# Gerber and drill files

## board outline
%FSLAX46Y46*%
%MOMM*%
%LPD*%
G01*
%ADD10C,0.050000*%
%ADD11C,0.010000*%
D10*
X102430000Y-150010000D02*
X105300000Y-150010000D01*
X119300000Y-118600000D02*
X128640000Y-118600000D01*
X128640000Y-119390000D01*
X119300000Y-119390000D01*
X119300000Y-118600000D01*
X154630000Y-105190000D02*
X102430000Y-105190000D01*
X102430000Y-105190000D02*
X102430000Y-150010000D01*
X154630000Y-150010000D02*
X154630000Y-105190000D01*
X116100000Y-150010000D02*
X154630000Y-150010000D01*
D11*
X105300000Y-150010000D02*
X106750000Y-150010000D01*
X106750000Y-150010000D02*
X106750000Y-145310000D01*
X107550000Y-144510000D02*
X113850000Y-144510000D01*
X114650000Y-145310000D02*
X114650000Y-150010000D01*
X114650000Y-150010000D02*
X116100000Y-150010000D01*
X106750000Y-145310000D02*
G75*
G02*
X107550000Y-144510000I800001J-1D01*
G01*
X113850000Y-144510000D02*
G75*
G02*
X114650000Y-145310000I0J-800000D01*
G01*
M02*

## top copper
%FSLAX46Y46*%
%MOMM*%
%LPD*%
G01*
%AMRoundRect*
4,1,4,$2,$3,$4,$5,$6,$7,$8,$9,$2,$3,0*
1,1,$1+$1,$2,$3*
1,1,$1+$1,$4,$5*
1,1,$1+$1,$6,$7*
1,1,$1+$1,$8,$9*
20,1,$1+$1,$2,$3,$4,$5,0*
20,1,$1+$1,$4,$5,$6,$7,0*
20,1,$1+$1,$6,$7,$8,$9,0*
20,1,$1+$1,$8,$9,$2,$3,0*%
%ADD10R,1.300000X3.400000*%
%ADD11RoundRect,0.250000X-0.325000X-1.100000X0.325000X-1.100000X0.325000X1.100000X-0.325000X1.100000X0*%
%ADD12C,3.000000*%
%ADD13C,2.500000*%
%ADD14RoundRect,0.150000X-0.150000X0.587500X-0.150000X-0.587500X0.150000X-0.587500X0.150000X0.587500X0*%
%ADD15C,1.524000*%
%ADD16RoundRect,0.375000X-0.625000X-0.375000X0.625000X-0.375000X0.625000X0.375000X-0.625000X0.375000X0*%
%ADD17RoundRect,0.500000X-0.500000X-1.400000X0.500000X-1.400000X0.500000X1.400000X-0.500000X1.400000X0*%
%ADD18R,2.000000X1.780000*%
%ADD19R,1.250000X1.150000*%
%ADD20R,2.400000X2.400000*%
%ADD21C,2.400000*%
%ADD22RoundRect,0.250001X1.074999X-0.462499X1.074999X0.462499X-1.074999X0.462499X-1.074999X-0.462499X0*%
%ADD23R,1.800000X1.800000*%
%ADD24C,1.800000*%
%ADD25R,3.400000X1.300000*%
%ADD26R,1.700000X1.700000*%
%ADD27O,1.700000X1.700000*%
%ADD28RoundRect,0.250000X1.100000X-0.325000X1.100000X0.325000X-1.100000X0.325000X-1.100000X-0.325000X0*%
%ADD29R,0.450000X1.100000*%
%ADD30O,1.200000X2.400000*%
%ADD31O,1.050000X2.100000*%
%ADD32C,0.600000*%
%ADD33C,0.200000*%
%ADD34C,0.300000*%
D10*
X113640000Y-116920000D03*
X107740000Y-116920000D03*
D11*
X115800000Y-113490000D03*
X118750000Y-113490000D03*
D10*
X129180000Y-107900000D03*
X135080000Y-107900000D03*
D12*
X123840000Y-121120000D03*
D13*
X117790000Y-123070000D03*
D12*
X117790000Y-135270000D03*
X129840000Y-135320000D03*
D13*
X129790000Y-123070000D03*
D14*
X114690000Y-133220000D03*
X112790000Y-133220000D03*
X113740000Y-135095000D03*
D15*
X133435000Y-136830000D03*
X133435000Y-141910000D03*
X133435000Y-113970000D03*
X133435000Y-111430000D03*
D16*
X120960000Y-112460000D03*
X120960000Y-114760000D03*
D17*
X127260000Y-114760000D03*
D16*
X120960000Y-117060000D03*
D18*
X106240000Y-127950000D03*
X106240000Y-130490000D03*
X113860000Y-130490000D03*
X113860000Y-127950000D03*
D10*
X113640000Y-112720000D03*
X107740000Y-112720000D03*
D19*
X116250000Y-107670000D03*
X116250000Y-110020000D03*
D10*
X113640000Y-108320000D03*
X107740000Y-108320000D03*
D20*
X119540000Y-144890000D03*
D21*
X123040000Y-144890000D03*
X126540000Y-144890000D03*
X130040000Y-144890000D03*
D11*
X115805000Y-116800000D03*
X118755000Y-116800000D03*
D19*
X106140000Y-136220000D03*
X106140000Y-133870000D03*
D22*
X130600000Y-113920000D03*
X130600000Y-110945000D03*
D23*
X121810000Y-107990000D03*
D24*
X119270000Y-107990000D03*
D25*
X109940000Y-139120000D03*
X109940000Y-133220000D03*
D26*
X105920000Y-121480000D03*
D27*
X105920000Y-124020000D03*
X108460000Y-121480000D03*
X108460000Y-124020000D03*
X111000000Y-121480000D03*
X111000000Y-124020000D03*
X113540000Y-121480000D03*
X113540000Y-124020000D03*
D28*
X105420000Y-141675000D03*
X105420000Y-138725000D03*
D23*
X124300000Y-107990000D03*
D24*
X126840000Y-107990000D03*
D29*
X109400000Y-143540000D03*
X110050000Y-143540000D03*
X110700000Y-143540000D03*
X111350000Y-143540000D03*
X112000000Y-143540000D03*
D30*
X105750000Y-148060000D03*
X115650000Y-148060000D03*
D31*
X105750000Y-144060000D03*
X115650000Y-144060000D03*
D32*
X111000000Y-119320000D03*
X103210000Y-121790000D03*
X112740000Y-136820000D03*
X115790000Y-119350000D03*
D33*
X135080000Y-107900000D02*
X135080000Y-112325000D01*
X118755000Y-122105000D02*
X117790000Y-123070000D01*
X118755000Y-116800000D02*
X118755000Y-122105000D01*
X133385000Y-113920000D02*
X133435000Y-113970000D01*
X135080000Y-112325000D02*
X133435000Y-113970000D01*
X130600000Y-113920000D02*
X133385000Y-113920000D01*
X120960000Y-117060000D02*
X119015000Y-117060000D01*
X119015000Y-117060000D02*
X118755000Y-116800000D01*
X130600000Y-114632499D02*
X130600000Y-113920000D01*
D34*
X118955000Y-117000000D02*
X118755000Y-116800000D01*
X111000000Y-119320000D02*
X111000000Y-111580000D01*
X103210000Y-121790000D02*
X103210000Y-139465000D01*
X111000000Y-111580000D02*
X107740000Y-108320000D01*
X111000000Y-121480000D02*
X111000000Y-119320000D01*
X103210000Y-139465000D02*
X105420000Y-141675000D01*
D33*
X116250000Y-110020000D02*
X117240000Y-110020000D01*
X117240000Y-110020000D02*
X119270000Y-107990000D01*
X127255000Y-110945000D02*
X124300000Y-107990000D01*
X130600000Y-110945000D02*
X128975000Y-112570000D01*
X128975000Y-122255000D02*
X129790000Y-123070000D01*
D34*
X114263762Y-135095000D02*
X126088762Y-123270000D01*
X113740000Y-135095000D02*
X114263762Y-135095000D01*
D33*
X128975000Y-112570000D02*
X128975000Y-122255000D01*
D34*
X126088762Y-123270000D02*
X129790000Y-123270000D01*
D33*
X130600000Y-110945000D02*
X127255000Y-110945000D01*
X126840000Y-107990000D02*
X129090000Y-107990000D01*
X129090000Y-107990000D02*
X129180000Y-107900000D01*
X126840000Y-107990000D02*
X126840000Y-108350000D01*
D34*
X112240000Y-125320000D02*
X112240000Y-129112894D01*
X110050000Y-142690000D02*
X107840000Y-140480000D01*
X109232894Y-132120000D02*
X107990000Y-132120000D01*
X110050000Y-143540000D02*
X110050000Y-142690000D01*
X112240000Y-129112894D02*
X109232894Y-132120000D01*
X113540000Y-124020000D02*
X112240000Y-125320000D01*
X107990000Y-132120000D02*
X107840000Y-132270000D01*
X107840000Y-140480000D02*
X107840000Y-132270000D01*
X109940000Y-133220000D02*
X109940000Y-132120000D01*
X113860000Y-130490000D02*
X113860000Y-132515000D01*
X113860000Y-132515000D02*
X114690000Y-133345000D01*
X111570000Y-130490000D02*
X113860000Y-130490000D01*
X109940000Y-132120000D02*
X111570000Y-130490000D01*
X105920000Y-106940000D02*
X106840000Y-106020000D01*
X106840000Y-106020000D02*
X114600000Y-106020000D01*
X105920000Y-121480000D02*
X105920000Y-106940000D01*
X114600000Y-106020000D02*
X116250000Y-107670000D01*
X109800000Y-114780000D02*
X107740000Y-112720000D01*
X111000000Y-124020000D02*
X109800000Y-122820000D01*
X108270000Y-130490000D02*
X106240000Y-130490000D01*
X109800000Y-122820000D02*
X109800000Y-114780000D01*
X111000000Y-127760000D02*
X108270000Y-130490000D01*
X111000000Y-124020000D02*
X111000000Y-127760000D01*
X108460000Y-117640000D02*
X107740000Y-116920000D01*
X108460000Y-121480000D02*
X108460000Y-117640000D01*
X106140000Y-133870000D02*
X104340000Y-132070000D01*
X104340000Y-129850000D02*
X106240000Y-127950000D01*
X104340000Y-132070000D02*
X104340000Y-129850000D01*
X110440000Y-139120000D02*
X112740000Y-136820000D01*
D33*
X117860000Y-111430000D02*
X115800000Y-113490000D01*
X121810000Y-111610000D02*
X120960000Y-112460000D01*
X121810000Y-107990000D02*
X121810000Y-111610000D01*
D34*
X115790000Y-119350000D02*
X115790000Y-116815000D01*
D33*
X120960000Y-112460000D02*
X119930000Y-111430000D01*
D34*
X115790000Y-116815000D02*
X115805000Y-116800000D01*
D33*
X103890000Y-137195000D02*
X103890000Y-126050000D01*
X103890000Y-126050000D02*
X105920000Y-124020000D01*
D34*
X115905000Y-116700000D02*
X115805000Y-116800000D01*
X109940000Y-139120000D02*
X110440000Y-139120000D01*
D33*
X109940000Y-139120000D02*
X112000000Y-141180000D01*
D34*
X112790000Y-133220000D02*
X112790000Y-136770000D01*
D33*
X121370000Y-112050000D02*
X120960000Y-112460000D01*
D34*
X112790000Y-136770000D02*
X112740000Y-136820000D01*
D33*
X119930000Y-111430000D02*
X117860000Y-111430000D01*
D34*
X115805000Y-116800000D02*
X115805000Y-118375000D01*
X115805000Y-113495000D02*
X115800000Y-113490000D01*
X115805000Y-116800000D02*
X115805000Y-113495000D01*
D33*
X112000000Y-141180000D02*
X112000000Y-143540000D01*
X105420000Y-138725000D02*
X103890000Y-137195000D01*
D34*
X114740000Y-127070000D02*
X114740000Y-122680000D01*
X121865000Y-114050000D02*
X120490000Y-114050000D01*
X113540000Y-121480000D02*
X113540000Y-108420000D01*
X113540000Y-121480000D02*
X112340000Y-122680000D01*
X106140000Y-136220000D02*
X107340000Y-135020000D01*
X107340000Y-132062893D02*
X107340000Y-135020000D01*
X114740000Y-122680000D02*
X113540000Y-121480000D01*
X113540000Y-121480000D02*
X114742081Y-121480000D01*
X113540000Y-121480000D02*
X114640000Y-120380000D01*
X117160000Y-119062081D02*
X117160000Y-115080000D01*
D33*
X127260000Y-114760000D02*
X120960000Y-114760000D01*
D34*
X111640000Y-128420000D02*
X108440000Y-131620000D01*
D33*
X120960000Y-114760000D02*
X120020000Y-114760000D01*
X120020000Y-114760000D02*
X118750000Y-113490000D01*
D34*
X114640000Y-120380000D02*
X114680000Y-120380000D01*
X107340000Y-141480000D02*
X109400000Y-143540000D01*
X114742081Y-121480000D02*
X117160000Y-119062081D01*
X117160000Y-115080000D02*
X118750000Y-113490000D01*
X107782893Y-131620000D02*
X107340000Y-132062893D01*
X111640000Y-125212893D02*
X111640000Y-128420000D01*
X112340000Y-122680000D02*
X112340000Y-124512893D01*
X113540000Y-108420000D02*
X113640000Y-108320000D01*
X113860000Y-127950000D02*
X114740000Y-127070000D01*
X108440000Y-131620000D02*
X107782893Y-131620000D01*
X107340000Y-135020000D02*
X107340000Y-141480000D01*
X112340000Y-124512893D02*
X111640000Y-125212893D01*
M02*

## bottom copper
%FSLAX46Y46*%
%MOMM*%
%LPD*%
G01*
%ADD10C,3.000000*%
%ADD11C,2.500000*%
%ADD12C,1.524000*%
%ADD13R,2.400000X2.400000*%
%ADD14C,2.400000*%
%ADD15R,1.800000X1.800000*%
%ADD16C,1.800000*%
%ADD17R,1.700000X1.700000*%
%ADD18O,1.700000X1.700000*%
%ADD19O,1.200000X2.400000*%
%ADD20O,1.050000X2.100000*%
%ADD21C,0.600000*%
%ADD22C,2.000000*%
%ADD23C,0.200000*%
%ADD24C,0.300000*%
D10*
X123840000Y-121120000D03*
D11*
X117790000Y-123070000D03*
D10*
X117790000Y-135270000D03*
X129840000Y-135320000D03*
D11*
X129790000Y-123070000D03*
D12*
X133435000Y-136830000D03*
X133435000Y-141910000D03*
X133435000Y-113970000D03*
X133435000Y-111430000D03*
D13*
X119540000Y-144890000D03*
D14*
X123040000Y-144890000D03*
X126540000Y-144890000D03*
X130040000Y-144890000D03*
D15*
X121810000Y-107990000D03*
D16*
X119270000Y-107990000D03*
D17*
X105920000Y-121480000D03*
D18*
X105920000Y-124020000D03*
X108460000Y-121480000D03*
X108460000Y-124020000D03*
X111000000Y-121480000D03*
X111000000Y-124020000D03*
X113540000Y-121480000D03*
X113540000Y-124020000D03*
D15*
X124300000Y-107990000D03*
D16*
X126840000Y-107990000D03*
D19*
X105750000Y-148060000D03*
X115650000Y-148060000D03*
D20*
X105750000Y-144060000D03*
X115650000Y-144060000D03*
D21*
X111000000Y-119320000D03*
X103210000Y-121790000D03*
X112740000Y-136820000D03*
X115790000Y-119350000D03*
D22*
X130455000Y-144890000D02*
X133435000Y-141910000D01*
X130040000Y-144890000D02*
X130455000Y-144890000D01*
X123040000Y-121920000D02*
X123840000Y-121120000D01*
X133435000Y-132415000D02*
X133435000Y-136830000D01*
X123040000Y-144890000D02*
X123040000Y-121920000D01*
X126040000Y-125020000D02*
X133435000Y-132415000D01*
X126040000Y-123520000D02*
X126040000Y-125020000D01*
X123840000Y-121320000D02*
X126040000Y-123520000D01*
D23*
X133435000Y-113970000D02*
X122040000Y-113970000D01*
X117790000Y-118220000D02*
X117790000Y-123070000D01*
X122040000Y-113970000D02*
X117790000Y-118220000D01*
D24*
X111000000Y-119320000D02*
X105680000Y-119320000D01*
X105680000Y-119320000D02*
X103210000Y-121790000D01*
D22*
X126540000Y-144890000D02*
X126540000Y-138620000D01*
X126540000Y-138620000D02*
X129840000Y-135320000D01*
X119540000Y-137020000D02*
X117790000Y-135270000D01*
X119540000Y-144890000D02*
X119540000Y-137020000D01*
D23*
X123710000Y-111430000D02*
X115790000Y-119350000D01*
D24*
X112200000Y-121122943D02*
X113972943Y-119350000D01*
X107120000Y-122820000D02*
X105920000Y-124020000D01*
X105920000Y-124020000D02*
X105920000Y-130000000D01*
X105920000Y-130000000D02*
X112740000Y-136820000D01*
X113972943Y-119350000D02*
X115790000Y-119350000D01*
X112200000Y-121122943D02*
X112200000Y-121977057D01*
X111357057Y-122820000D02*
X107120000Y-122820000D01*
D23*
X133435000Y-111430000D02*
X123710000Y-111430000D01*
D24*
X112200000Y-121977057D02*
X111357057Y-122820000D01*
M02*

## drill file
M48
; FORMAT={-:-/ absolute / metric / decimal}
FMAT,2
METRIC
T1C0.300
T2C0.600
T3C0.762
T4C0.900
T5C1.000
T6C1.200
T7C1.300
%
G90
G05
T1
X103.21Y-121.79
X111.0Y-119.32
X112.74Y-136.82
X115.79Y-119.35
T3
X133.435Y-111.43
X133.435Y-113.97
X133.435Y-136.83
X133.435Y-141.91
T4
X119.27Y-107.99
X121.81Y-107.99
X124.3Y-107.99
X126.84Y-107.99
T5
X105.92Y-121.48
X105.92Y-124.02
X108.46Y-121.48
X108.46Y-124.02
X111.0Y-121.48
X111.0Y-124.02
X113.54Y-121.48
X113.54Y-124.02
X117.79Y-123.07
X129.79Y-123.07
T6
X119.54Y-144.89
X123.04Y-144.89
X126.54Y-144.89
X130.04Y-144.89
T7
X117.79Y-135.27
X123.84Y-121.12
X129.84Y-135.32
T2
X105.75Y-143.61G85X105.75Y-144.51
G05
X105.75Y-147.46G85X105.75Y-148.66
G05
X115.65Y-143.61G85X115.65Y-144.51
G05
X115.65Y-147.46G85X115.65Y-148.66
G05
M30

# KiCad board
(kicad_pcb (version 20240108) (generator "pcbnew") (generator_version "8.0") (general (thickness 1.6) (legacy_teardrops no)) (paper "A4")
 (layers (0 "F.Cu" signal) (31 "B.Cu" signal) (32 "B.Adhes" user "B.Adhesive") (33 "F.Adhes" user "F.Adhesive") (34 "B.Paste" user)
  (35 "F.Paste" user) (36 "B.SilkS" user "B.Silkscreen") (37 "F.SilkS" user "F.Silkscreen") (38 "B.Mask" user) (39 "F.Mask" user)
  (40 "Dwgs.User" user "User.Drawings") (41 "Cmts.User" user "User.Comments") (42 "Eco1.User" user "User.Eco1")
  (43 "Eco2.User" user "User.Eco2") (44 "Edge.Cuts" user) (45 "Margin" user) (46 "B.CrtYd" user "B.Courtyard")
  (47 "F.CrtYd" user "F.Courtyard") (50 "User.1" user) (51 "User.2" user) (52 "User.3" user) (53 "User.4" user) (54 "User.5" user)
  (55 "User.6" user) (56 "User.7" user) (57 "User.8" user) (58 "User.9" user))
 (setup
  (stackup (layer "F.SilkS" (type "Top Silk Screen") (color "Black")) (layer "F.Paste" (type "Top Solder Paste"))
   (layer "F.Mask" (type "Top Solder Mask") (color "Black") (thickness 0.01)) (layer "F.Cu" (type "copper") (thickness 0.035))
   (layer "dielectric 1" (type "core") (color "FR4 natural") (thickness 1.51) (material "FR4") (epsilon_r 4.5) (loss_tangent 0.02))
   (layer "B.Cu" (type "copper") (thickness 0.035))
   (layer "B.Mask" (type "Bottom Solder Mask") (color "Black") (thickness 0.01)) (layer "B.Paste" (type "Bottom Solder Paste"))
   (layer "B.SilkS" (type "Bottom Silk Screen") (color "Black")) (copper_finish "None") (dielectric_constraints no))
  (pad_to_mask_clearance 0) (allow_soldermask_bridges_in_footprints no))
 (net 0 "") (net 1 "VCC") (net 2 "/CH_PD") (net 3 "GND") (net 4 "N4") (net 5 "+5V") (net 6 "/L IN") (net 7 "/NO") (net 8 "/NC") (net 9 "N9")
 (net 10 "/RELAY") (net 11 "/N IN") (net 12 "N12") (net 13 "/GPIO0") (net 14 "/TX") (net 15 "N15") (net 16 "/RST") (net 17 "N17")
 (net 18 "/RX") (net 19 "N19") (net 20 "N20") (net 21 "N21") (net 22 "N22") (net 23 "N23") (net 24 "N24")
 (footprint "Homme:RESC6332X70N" (layer "F.Cu") (at 110.69 116.92 180)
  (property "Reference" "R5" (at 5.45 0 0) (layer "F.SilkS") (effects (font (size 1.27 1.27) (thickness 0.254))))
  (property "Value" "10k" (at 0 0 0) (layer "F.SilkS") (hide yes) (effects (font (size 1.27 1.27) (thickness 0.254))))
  (pad "1" smd rect (at -2.95 0 180) (size 1.3 3.4) (layers "F.Cu" "F.Paste" "F.Mask") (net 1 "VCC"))
  (pad "2" smd rect (at 2.95 0 180) (size 1.3 3.4) (layers "F.Cu" "F.Paste" "F.Mask") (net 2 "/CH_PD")))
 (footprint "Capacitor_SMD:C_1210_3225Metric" (layer "F.Cu") (at 117.275 113.49)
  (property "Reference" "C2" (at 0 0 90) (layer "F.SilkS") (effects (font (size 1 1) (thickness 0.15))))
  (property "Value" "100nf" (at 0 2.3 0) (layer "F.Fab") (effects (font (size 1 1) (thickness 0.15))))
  (pad "1" smd roundrect (at -1.475 0) (size 1.15 2.7) (layers "F.Cu" "F.Paste" "F.Mask") (roundrect_rratio 0.217391) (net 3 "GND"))
  (pad "2" smd roundrect (at 1.475 0) (size 1.15 2.7) (layers "F.Cu" "F.Paste" "F.Mask") (roundrect_rratio 0.217391) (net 1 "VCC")))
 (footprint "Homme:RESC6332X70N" (layer "F.Cu") (at 132.13 107.9)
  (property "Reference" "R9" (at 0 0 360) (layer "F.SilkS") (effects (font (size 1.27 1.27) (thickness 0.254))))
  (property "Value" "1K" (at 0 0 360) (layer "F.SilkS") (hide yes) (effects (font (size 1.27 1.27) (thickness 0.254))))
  (pad "1" smd rect (at -2.95 0) (size 1.3 3.4) (layers "F.Cu" "F.Paste" "F.Mask") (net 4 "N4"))
  (pad "2" smd rect (at 2.95 0) (size 1.3 3.4) (layers "F.Cu" "F.Paste" "F.Mask") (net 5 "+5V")))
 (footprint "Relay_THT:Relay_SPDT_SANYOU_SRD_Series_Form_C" (layer "F.Cu") (at 123.84 121.12 -90)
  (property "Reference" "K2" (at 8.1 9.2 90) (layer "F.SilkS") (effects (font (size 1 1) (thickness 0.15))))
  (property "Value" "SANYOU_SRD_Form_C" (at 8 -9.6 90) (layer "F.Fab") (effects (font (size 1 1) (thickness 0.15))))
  (pad "1" thru_hole circle (at 0 0) (size 3 3) (drill 1.3) (layers "*.Cu" "*.Mask") (remove_unused_layers no) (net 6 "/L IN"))
  (pad "2" thru_hole circle (at 1.95 6.05) (size 2.5 2.5) (drill 1) (layers "*.Cu" "*.Mask") (remove_unused_layers no) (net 5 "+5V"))
  (pad "3" thru_hole circle (at 14.15 6.05) (size 3 3) (drill 1.3) (layers "*.Cu" "*.Mask") (remove_unused_layers no) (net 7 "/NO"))
  (pad "4" thru_hole circle (at 14.2 -6) (size 3 3) (drill 1.3) (layers "*.Cu" "*.Mask") (remove_unused_layers no) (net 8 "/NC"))
  (pad "5" thru_hole circle (at 1.95 -5.95) (size 2.5 2.5) (drill 1) (layers "*.Cu" "*.Mask") (remove_unused_layers no) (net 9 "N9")))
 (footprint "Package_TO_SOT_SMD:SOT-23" (layer "F.Cu") (at 113.74 134.1575 -90)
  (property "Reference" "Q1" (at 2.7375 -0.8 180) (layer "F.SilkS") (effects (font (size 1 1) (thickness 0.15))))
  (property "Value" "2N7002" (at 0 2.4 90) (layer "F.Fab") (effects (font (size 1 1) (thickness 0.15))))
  (pad "1" smd roundrect (at -0.9375 -0.95 270) (size 1.475 0.6) (layers "F.Cu" "F.Paste" "F.Mask") (roundrect_rratio 0.25)
   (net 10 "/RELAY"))
  (pad "2" smd roundrect (at -0.9375 0.95 270) (size 1.475 0.6) (layers "F.Cu" "F.Paste" "F.Mask") (roundrect_rratio 0.25) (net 3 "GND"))
  (pad "3" smd roundrect (at 0.9375 0 270) (size 1.475 0.6) (layers "F.Cu" "F.Paste" "F.Mask") (roundrect_rratio 0.25) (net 9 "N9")))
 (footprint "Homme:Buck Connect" (layer "F.Cu") (at 132.435 126.47 -90)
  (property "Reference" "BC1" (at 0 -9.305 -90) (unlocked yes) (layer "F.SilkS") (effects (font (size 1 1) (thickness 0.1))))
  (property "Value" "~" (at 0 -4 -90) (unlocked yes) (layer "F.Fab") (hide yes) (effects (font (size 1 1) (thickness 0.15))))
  (pad "1" thru_hole circle (at 10.36 -1 270) (size 1.524 1.524) (drill 0.762) (layers "*.Cu" "*.Mask") (remove_unused_layers no)
   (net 6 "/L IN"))
  (pad "2" thru_hole circle (at 15.44 -1 270) (size 1.524 1.524) (drill 0.762) (layers "*.Cu" "*.Mask") (remove_unused_layers no)
   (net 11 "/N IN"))
  (pad "3" thru_hole circle (at -12.5 -1 270) (size 1.524 1.524) (drill 0.762) (layers "*.Cu" "*.Mask") (remove_unused_layers no)
   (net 5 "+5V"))
  (pad "4" thru_hole circle (at -15.04 -1 270) (size 1.524 1.524) (drill 0.762) (layers "*.Cu" "*.Mask") (remove_unused_layers no)
   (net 3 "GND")))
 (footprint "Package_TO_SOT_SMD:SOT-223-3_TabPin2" (layer "F.Cu") (at 124.11 114.76)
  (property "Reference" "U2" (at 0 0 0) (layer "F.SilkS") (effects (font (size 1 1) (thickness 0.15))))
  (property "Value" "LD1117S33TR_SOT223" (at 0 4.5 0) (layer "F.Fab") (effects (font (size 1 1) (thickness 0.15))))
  (pad "1" smd roundrect (at -3.15 -2.3) (size 2 1.5) (layers "F.Cu" "F.Paste" "F.Mask") (roundrect_rratio 0.25) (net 3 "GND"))
  (pad "2" smd roundrect (at -3.15 0) (size 2 1.5) (layers "F.Cu" "F.Paste" "F.Mask") (roundrect_rratio 0.25) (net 1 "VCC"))
  (pad "2" smd roundrect (at 3.15 0) (size 2 3.8) (layers "F.Cu" "F.Paste" "F.Mask") (roundrect_rratio 0.25) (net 1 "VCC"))
  (pad "3" smd roundrect (at -3.15 2.3) (size 2 1.5) (layers "F.Cu" "F.Paste" "F.Mask") (roundrect_rratio 0.25) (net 5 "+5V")))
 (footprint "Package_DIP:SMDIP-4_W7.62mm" (layer "F.Cu") (at 110.05 129.22)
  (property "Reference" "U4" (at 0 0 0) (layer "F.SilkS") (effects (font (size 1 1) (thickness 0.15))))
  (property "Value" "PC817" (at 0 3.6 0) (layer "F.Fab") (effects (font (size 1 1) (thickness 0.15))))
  (pad "1" smd rect (at -3.81 -1.27) (size 2 1.78) (layers "F.Cu" "F.Paste" "F.Mask") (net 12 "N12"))
  (pad "2" smd rect (at -3.81 1.27) (size 2 1.78) (layers "F.Cu" "F.Paste" "F.Mask") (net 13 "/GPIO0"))
  (pad "3" smd rect (at 3.81 1.27) (size 2 1.78) (layers "F.Cu" "F.Paste" "F.Mask") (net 10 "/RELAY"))
  (pad "4" smd rect (at 3.81 -1.27) (size 2 1.78) (layers "F.Cu" "F.Paste" "F.Mask") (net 1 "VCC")))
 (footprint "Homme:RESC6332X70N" (layer "F.Cu") (at 110.69 112.72 180)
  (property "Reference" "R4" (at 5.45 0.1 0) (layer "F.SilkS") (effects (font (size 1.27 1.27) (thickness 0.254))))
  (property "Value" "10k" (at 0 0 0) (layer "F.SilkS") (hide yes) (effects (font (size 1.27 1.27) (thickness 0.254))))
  (pad "1" smd rect (at -2.95 0 180) (size 1.3 3.4) (layers "F.Cu" "F.Paste" "F.Mask") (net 1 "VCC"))
  (pad "2" smd rect (at 2.95 0 180) (size 1.3 3.4) (layers "F.Cu" "F.Paste" "F.Mask") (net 13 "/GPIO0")))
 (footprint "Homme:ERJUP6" (layer "F.Cu") (at 116.25 108.845 -90)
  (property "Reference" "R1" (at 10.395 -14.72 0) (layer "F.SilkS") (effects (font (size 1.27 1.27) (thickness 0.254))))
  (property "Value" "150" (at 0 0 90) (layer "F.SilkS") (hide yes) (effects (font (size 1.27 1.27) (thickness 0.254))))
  (pad "1" smd rect (at -1.175 0 270) (size 1.15 1.25) (layers "F.Cu" "F.Paste" "F.Mask") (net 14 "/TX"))
  (pad "2" smd rect (at 1.175 0 270) (size 1.15 1.25) (layers "F.Cu" "F.Paste" "F.Mask") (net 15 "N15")))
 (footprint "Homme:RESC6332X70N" (layer "F.Cu") (at 110.69 108.32 180)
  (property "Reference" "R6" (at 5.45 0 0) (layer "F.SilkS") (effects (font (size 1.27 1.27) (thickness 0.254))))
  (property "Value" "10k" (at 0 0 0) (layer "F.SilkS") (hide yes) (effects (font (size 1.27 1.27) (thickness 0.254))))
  (pad "1" smd rect (at -2.95 0 180) (size 1.3 3.4) (layers "F.Cu" "F.Paste" "F.Mask") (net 1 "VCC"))
  (pad "2" smd rect (at 2.95 0 180) (size 1.3 3.4) (layers "F.Cu" "F.Paste" "F.Mask") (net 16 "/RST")))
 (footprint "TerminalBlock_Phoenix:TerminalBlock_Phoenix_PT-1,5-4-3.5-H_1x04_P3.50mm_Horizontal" (layer "F.Cu") (at 119.54 144.89)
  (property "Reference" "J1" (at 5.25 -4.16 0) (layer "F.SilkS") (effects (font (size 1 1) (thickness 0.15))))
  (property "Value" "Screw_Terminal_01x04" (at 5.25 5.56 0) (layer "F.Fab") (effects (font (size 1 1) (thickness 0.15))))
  (pad "1" thru_hole rect (at 0 0) (size 2.4 2.4) (drill 1.2) (layers "*.Cu" "*.Mask") (remove_unused_layers no) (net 7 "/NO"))
  (pad "2" thru_hole circle (at 3.5 0) (size 2.4 2.4) (drill 1.2) (layers "*.Cu" "*.Mask") (remove_unused_layers no) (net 6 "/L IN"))
  (pad "3" thru_hole circle (at 7 0) (size 2.4 2.4) (drill 1.2) (layers "*.Cu" "*.Mask") (remove_unused_layers no) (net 8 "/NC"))
  (pad "4" thru_hole circle (at 10.5 0) (size 2.4 2.4) (drill 1.2) (layers "*.Cu" "*.Mask") (remove_unused_layers no) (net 11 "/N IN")))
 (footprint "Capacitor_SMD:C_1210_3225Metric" (layer "F.Cu") (at 117.28 116.8)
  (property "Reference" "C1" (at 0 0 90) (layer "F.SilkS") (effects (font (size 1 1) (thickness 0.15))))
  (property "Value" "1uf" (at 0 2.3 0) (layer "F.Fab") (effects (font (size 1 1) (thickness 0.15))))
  (pad "1" smd roundrect (at -1.475 0) (size 1.15 2.7) (layers "F.Cu" "F.Paste" "F.Mask") (roundrect_rratio 0.217391) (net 3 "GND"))
  (pad "2" smd roundrect (at 1.475 0) (size 1.15 2.7) (layers "F.Cu" "F.Paste" "F.Mask") (roundrect_rratio 0.217391) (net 5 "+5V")))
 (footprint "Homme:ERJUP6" (layer "F.Cu") (at 106.14 135.045 90)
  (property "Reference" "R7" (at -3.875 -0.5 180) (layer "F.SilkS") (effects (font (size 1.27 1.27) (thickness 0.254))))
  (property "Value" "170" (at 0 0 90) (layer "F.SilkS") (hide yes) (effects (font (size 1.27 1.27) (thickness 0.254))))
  (pad "1" smd rect (at -1.175 0 90) (size 1.15 1.25) (layers "F.Cu" "F.Paste" "F.Mask") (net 1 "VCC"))
  (pad "2" smd rect (at 1.175 0 90) (size 1.15 1.25) (layers "F.Cu" "F.Paste" "F.Mask") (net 12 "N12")))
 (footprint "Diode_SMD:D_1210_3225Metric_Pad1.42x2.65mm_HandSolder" (layer "F.Cu") (at 130.6 112.4325 90)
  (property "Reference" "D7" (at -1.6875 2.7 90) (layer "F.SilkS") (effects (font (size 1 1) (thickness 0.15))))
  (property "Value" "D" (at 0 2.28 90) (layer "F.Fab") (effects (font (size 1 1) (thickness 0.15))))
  (pad "1" smd roundrect (at -1.4875 0 90) (size 1.425 2.65) (layers "F.Cu" "F.Paste" "F.Mask") (roundrect_rratio 0.175439) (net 5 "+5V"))
  (pad "2" smd roundrect (at 1.4875 0 90) (size 1.425 2.65) (layers "F.Cu" "F.Paste" "F.Mask") (roundrect_rratio 0.175439) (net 9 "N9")))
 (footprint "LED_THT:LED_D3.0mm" (layer "F.Cu") (at 121.81 107.99 180)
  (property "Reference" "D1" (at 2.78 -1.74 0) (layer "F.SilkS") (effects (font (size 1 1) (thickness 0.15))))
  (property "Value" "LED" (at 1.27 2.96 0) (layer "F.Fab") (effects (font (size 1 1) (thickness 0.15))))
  (pad "1" thru_hole rect (at 0 0 180) (size 1.8 1.8) (drill 0.9) (layers "*.Cu" "*.Mask") (remove_unused_layers no) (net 3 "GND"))
  (pad "2" thru_hole circle (at 2.54 0 180) (size 1.8 1.8) (drill 0.9) (layers "*.Cu" "*.Mask") (remove_unused_layers no) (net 15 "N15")))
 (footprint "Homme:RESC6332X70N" (layer "F.Cu") (at 109.94 136.17 90)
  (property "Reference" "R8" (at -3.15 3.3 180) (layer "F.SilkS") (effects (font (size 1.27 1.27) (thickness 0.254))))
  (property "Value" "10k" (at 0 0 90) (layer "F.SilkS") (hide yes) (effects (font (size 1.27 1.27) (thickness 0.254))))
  (pad "1" smd rect (at -2.95 0 90) (size 1.3 3.4) (layers "F.Cu" "F.Paste" "F.Mask") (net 3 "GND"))
  (pad "2" smd rect (at 2.95 0 90) (size 1.3 3.4) (layers "F.Cu" "F.Paste" "F.Mask") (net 10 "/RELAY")))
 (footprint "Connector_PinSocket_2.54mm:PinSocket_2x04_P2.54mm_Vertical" (layer "F.Cu") (at 105.92 121.48 90)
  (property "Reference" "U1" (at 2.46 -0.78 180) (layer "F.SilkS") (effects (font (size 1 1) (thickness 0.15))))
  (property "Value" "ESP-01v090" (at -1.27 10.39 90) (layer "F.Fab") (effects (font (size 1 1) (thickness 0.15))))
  (pad "1" thru_hole rect (at 0 0 90) (size 1.7 1.7) (drill 1) (layers "*.Cu" "*.Mask") (remove_unused_layers no) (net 14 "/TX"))
  (pad "2" thru_hole oval (at -2.54 0 90) (size 1.7 1.7) (drill 1) (layers "*.Cu" "*.Mask") (remove_unused_layers no) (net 3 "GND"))
  (pad "3" thru_hole oval (at 0 2.54 90) (size 1.7 1.7) (drill 1) (layers "*.Cu" "*.Mask") (remove_unused_layers no) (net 2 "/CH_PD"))
  (pad "4" thru_hole oval (at -2.54 2.54 90) (size 1.7 1.7) (drill 1) (layers "*.Cu" "*.Mask") (remove_unused_layers no) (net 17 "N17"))
  (pad "5" thru_hole oval (at 0 5.08 90) (size 1.7 1.7) (drill 1) (layers "*.Cu" "*.Mask") (remove_unused_layers no) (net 16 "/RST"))
  (pad "6" thru_hole oval (at -2.54 5.08 90) (size 1.7 1.7) (drill 1) (layers "*.Cu" "*.Mask") (remove_unused_layers no) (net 13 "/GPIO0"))
  (pad "7" thru_hole oval (at 0 7.62 90) (size 1.7 1.7) (drill 1) (layers "*.Cu" "*.Mask") (remove_unused_layers no) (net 1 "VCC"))
  (pad "8" thru_hole oval (at -2.54 7.62 90) (size 1.7 1.7) (drill 1) (layers "*.Cu" "*.Mask") (remove_unused_layers no) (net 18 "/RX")))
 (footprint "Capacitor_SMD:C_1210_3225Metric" (layer "F.Cu") (at 105.42 140.2 90)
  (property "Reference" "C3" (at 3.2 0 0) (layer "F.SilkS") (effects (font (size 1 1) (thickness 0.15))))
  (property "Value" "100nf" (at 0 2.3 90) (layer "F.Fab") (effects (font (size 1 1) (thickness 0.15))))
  (pad "1" smd roundrect (at -1.475 0 90) (size 1.15 2.7) (layers "F.Cu" "F.Paste" "F.Mask") (roundrect_rratio 0.217391) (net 16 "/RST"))
  (pad "2" smd roundrect (at 1.475 0 90) (size 1.15 2.7) (layers "F.Cu" "F.Paste" "F.Mask") (roundrect_rratio 0.217391) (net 3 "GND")))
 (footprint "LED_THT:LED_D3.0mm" (layer "F.Cu") (at 124.3 107.99)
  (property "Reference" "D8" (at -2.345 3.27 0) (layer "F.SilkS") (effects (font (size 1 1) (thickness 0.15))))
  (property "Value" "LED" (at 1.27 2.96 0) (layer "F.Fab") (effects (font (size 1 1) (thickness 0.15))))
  (pad "1" thru_hole rect (at 0 0) (size 1.8 1.8) (drill 0.9) (layers "*.Cu" "*.Mask") (remove_unused_layers no) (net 9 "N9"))
  (pad "2" thru_hole circle (at 2.54 0) (size 1.8 1.8) (drill 0.9) (layers "*.Cu" "*.Mask") (remove_unused_layers no) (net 4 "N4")))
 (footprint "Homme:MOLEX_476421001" (layer "F.Cu") (at 110.7 146.825)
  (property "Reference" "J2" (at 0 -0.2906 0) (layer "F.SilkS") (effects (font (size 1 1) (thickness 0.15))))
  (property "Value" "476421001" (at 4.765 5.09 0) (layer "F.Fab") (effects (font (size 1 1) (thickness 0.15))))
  (fp_line (start -5.4 3.185) (end -3.95 3.185) (stroke (width 0.01) (type solid)) (layer "Edge.Cuts"))
  (fp_line (start -3.95 3.185) (end -3.95 -1.515) (stroke (width 0.01) (type solid)) (layer "Edge.Cuts"))
  (fp_line (start -3.15 -2.315) (end 3.15 -2.315) (stroke (width 0.01) (type solid)) (layer "Edge.Cuts"))
  (fp_line (start 3.95 -1.515) (end 3.95 3.185) (stroke (width 0.01) (type solid)) (layer "Edge.Cuts"))
  (fp_line (start 3.95 3.185) (end 5.4 3.185) (stroke (width 0.01) (type solid)) (layer "Edge.Cuts"))
  (fp_arc (start -3.95 -1.515) (mid -3.715685 -2.080685) (end -3.15 -2.315) (stroke (width 0.01) (type solid)) (layer "Edge.Cuts"))
  (fp_arc (start 3.15 -2.315) (mid 3.715685 -2.080685) (end 3.95 -1.515) (stroke (width 0.01) (type solid)) (layer "Edge.Cuts"))
  (pad "1" smd rect (at -1.3 -3.285) (size 0.45 1.1) (layers "F.Cu" "F.Paste" "F.Mask") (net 1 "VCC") (solder_mask_margin 0.0762))
  (pad "2" smd rect (at -0.65 -3.285) (size 0.45 1.1) (layers "F.Cu" "F.Paste" "F.Mask") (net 18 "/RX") (solder_mask_margin 0.0762))
  (pad "3" smd rect (at 0 -3.285) (size 0.45 1.1) (layers "F.Cu" "F.Paste" "F.Mask") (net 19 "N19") (solder_mask_margin 0.0762))
  (pad "4" smd rect (at 0.65 -3.285) (size 0.45 1.1) (layers "F.Cu" "F.Paste" "F.Mask") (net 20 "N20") (solder_mask_margin 0.0762))
  (pad "5" smd rect (at 1.3 -3.285) (size 0.45 1.1) (layers "F.Cu" "F.Paste" "F.Mask") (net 3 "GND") (solder_mask_margin 0.0762))
  (pad "P1" thru_hole oval (at -4.95 1.235) (size 1.2 2.4) (drill oval 0.6 1.8) (layers "*.Cu" "*.Mask") (remove_unused_layers no)
   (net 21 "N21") (solder_mask_margin 0.0762))
  (pad "P2" thru_hole oval (at 4.95 1.235) (size 1.2 2.4) (drill oval 0.6 1.8) (layers "*.Cu" "*.Mask") (remove_unused_layers no)
   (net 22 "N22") (solder_mask_margin 0.0762))
  (pad "P3" thru_hole oval (at -4.95 -2.765) (size 1.05 2.1) (drill oval 0.6 1.5) (layers "*.Cu" "*.Mask") (remove_unused_layers no)
   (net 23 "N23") (solder_mask_margin 0.0762))
  (pad "P4" thru_hole oval (at 4.95 -2.765) (size 1.05 2.1) (drill oval 0.6 1.5) (layers "*.Cu" "*.Mask") (remove_unused_layers no)
   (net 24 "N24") (solder_mask_margin 0.0762)))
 (gr_line (start 102.43 150.01) (end 105.3 150.01) (stroke (width 0.05) (type default)) (layer "Edge.Cuts"))
 (gr_rect (start 119.3 118.6) (end 128.64 119.39) (stroke (width 0.05) (type default)) (fill none) (layer "Edge.Cuts"))
 (gr_line (start 154.63 105.19) (end 102.43 105.19) (stroke (width 0.05) (type default)) (layer "Edge.Cuts"))
 (gr_line (start 102.43 105.19) (end 102.43 150.01) (stroke (width 0.05) (type default)) (layer "Edge.Cuts"))
 (gr_line (start 154.63 150.01) (end 154.63 105.19) (stroke (width 0.05) (type default)) (layer "Edge.Cuts"))
 (gr_line (start 116.1 150.01) (end 154.63 150.01) (stroke (width 0.05) (type default)) (layer "Edge.Cuts"))
 (segment (start 130.455 144.89) (end 133.435 141.91) (width 2) (layer "B.Cu") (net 11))
 (segment (start 130.04 144.89) (end 130.455 144.89) (width 2) (layer "B.Cu") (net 11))
 (segment (start 123.04 121.92) (end 123.84 121.12) (width 2) (layer "B.Cu") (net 6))
 (segment (start 133.435 132.415) (end 133.435 136.83) (width 2) (layer "B.Cu") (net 6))
 (segment (start 123.04 144.89) (end 123.04 121.92) (width 2) (layer "B.Cu") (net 6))
 (segment (start 126.04 125.02) (end 133.435 132.415) (width 2) (layer "B.Cu") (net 6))
 (segment (start 126.04 123.52) (end 126.04 125.02) (width 2) (layer "B.Cu") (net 6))
 (segment (start 123.84 121.32) (end 126.04 123.52) (width 2) (layer "B.Cu") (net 6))
 (segment (start 135.08 107.9) (end 135.08 112.325) (width 0.2) (layer "F.Cu") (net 5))
 (segment (start 118.755 122.105) (end 117.79 123.07) (width 0.2) (layer "F.Cu") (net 5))
 (segment (start 118.755 116.8) (end 118.755 122.105) (width 0.2) (layer "F.Cu") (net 5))
 (segment (start 133.385 113.92) (end 133.435 113.97) (width 0.2) (layer "F.Cu") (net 5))
 (segment (start 135.08 112.325) (end 133.435 113.97) (width 0.2) (layer "F.Cu") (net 5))
 (segment (start 130.6 113.92) (end 133.385 113.92) (width 0.2) (layer "F.Cu") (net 5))
 (segment (start 120.96 117.06) (end 119.015 117.06) (width 0.2) (layer "F.Cu") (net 5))
 (segment (start 119.015 117.06) (end 118.755 116.8) (width 0.2) (layer "F.Cu") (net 5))
 (segment (start 130.6 114.632499) (end 130.6 113.92) (width 0.2) (layer "F.Cu") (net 5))
 (segment (start 118.955 117) (end 118.755 116.8) (width 0.3) (layer "F.Cu") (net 5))
 (segment (start 133.435 113.97) (end 122.04 113.97) (width 0.2) (layer "B.Cu") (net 5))
 (segment (start 117.79 118.22) (end 117.79 123.07) (width 0.2) (layer "B.Cu") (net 5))
 (segment (start 122.04 113.97) (end 117.79 118.22) (width 0.2) (layer "B.Cu") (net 5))
 (segment (start 111 119.32) (end 111 111.58) (width 0.3) (layer "F.Cu") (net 16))
 (segment (start 103.21 121.79) (end 103.21 139.465) (width 0.3) (layer "F.Cu") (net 16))
 (segment (start 111 111.58) (end 107.74 108.32) (width 0.3) (layer "F.Cu") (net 16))
 (segment (start 111 121.48) (end 111 119.32) (width 0.3) (layer "F.Cu") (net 16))
 (segment (start 103.21 139.465) (end 105.42 141.675) (width 0.3) (layer "F.Cu") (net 16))
 (via (at 111 119.32) (size 0.6) (drill 0.3) (layers "F.Cu" "B.Cu") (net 16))
 (via (at 103.21 121.79) (size 0.6) (drill 0.3) (layers "F.Cu" "B.Cu") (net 16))
 (segment (start 111 119.32) (end 105.68 119.32) (width 0.3) (layer "B.Cu") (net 16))
 (segment (start 105.68 119.32) (end 103.21 121.79) (width 0.3) (layer "B.Cu") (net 16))
 (segment (start 116.25 110.02) (end 117.24 110.02) (width 0.2) (layer "F.Cu") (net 15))
 (segment (start 117.24 110.02) (end 119.27 107.99) (width 0.2) (layer "F.Cu") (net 15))
 (segment (start 127.255 110.945) (end 124.3 107.99) (width 0.2) (layer "F.Cu") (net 9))
 (segment (start 130.6 110.945) (end 128.975 112.57) (width 0.2) (layer "F.Cu") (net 9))
 (segment (start 128.975 122.255) (end 129.79 123.07) (width 0.2) (layer "F.Cu") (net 9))
 (segment (start 114.263762 135.095) (end 126.088762 123.27) (width 0.3) (layer "F.Cu") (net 9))
 (segment (start 113.74 135.095) (end 114.263762 135.095) (width 0.3) (layer "F.Cu") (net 9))
 (segment (start 128.975 112.57) (end 128.975 122.255) (width 0.2) (layer "F.Cu") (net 9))
 (segment (start 126.088762 123.27) (end 129.79 123.27) (width 0.3) (layer "F.Cu") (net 9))
 (segment (start 130.6 110.945) (end 127.255 110.945) (width 0.2) (layer "F.Cu") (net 9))
 (segment (start 126.84 107.99) (end 129.09 107.99) (width 0.2) (layer "F.Cu") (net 4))
 (segment (start 129.09 107.99) (end 129.18 107.9) (width 0.2) (layer "F.Cu") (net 4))
 (segment (start 126.84 107.99) (end 126.84 108.35) (width 0.2) (layer "F.Cu") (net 4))
 (segment (start 112.24 125.32) (end 112.24 129.112894) (width 0.3) (layer "F.Cu") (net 18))
 (segment (start 110.05 142.69) (end 107.84 140.48) (width 0.3) (layer "F.Cu") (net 18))
 (segment (start 109.232894 132.12) (end 107.99 132.12) (width 0.3) (layer "F.Cu") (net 18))
 (segment (start 110.05 143.54) (end 110.05 142.69) (width 0.3) (layer "F.Cu") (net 18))
 (segment (start 112.24 129.112894) (end 109.232894 132.12) (width 0.3) (layer "F.Cu") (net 18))
 (segment (start 113.54 124.02) (end 112.24 125.32) (width 0.3) (layer "F.Cu") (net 18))
 (segment (start 107.99 132.12) (end 107.84 132.27) (width 0.3) (layer "F.Cu") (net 18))
 (segment (start 107.84 140.48) (end 107.84 132.27) (width 0.3) (layer "F.Cu") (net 18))
 (segment (start 126.54 144.89) (end 126.54 138.62) (width 2) (layer "B.Cu") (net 8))
 (segment (start 126.54 138.62) (end 129.84 135.32) (width 2) (layer "B.Cu") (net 8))
 (segment (start 119.54 137.02) (end 117.79 135.27) (width 2) (layer "B.Cu") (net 7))
 (segment (start 119.54 144.89) (end 119.54 137.02) (width 2) (layer "B.Cu") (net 7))
 (segment (start 109.94 133.22) (end 109.94 132.12) (width 0.3) (layer "F.Cu") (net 10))
 (segment (start 113.86 130.49) (end 113.86 132.515) (width 0.3) (layer "F.Cu") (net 10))
 (segment (start 113.86 132.515) (end 114.69 133.345) (width 0.3) (layer "F.Cu") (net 10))
 (segment (start 111.57 130.49) (end 113.86 130.49) (width 0.3) (layer "F.Cu") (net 10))
 (segment (start 109.94 132.12) (end 111.57 130.49) (width 0.3) (layer "F.Cu") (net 10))
 (segment (start 105.92 106.94) (end 106.84 106.02) (width 0.3) (layer "F.Cu") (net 14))
 (segment (start 106.84 106.02) (end 114.6 106.02) (width 0.3) (layer "F.Cu") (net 14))
 (segment (start 105.92 121.48) (end 105.92 106.94) (width 0.3) (layer "F.Cu") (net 14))
 (segment (start 114.6 106.02) (end 116.25 107.67) (width 0.3) (layer "F.Cu") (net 14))
 (segment (start 109.8 114.78) (end 107.74 112.72) (width 0.3) (layer "F.Cu") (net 13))
 (segment (start 111 124.02) (end 109.8 122.82) (width 0.3) (layer "F.Cu") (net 13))
 (segment (start 108.27 130.49) (end 106.24 130.49) (width 0.3) (layer "F.Cu") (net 13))
 (segment (start 109.8 122.82) (end 109.8 114.78) (width 0.3) (layer "F.Cu") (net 13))
 (segment (start 111 127.76) (end 108.27 130.49) (width 0.3) (layer "F.Cu") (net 13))
 (segment (start 111 124.02) (end 111 127.76) (width 0.3) (layer "F.Cu") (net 13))
 (segment (start 108.46 117.64) (end 107.74 116.92) (width 0.3) (layer "F.Cu") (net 2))
 (segment (start 108.46 121.48) (end 108.46 117.64) (width 0.3) (layer "F.Cu") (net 2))
 (segment (start 106.14 133.87) (end 104.34 132.07) (width 0.3) (layer "F.Cu") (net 12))
 (segment (start 104.34 129.85) (end 106.24 127.95) (width 0.3) (layer "F.Cu") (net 12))
 (segment (start 104.34 132.07) (end 104.34 129.85) (width 0.3) (layer "F.Cu") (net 12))
 (segment (start 110.44 139.12) (end 112.74 136.82) (width 0.3) (layer "F.Cu") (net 3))
 (segment (start 117.86 111.43) (end 115.8 113.49) (width 0.2) (layer "F.Cu") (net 3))
 (segment (start 121.81 111.61) (end 120.96 112.46) (width 0.2) (layer "F.Cu") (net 3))
 (segment (start 121.81 107.99) (end 121.81 111.61) (width 0.2) (layer "F.Cu") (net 3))
 (segment (start 115.79 119.35) (end 115.79 116.815) (width 0.3) (layer "F.Cu") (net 3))
 (segment (start 120.96 112.46) (end 119.93 111.43) (width 0.2) (layer "F.Cu") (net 3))
 (segment (start 115.79 116.815) (end 115.805 116.8) (width 0.3) (layer "F.Cu") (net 3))
 (segment (start 103.89 137.195) (end 103.89 126.05) (width 0.2) (layer "F.Cu") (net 3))
 (segment (start 103.89 126.05) (end 105.92 124.02) (width 0.2) (layer "F.Cu") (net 3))
 (segment (start 115.905 116.7) (end 115.805 116.8) (width 0.3) (layer "F.Cu") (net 3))
 (segment (start 109.94 139.12) (end 110.44 139.12) (width 0.3) (layer "F.Cu") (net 3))
 (segment (start 109.94 139.12) (end 112 141.18) (width 0.2) (layer "F.Cu") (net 3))
 (segment (start 112.79 133.22) (end 112.79 136.77) (width 0.3) (layer "F.Cu") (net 3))
 (segment (start 121.37 112.05) (end 120.96 112.46) (width 0.2) (layer "F.Cu") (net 3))
 (segment (start 112.79 136.77) (end 112.74 136.82) (width 0.3) (layer "F.Cu") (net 3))
 (segment (start 119.93 111.43) (end 117.86 111.43) (width 0.2) (layer "F.Cu") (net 3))
 (segment (start 115.805 116.8) (end 115.805 118.375) (width 0.3) (layer "F.Cu") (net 3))
 (segment (start 115.805 113.495) (end 115.8 113.49) (width 0.3) (layer "F.Cu") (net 3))
 (segment (start 115.805 116.8) (end 115.805 113.495) (width 0.3) (layer "F.Cu") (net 3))
 (segment (start 112 141.18) (end 112 143.54) (width 0.2) (layer "F.Cu") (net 3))
 (segment (start 105.42 138.725) (end 103.89 137.195) (width 0.2) (layer "F.Cu") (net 3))
 (via (at 112.74 136.82) (size 0.6) (drill 0.3) (layers "F.Cu" "B.Cu") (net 3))
 (via (at 115.79 119.35) (size 0.6) (drill 0.3) (layers "F.Cu" "B.Cu") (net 3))
 (segment (start 123.71 111.43) (end 115.79 119.35) (width 0.2) (layer "B.Cu") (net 3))
 (segment (start 112.2 121.122943) (end 113.972943 119.35) (width 0.3) (layer "B.Cu") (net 3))
 (segment (start 107.12 122.82) (end 105.92 124.02) (width 0.3) (layer "B.Cu") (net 3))
 (segment (start 105.92 124.02) (end 105.92 130) (width 0.3) (layer "B.Cu") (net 3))
 (segment (start 105.92 130) (end 112.74 136.82) (width 0.3) (layer "B.Cu") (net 3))
 (segment (start 113.972943 119.35) (end 115.79 119.35) (width 0.3) (layer "B.Cu") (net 3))
 (segment (start 112.2 121.122943) (end 112.2 121.977057) (width 0.3) (layer "B.Cu") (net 3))
 (segment (start 111.357057 122.82) (end 107.12 122.82) (width 0.3) (layer "B.Cu") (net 3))
 (segment (start 133.435 111.43) (end 123.71 111.43) (width 0.2) (layer "B.Cu") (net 3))
 (segment (start 112.2 121.977057) (end 111.357057 122.82) (width 0.3) (layer "B.Cu") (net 3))
 (segment (start 114.74 127.07) (end 114.74 122.68) (width 0.3) (layer "F.Cu") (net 1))
 (segment (start 121.865 114.05) (end 120.49 114.05) (width 0.3) (layer "F.Cu") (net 1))
 (segment (start 113.54 121.48) (end 113.54 108.42) (width 0.3) (layer "F.Cu") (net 1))
 (segment (start 113.54 121.48) (end 112.34 122.68) (width 0.3) (layer "F.Cu") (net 1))
 (segment (start 106.14 136.22) (end 107.34 135.02) (width 0.3) (layer "F.Cu") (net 1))
 (segment (start 107.34 132.062893) (end 107.34 135.02) (width 0.3) (layer "F.Cu") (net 1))
 (segment (start 114.74 122.68) (end 113.54 121.48) (width 0.3) (layer "F.Cu") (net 1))
 (segment (start 113.54 121.48) (end 114.742081 121.48) (width 0.3) (layer "F.Cu") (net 1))
 (segment (start 113.54 121.48) (end 114.64 120.38) (width 0.3) (layer "F.Cu") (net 1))
 (segment (start 117.16 119.062081) (end 117.16 115.08) (width 0.3) (layer "F.Cu") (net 1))
 (segment (start 127.26 114.76) (end 120.96 114.76) (width 0.2) (layer "F.Cu") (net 1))
 (segment (start 111.64 128.42) (end 108.44 131.62) (width 0.3) (layer "F.Cu") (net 1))
 (segment (start 120.96 114.76) (end 120.02 114.76) (width 0.2) (layer "F.Cu") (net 1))
 (segment (start 120.02 114.76) (end 118.75 113.49) (width 0.2) (layer "F.Cu") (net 1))
 (segment (start 114.64 120.38) (end 114.68 120.38) (width 0.3) (layer "F.Cu") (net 1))
 (segment (start 107.34 141.48) (end 109.4 143.54) (width 0.3) (layer "F.Cu") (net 1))
 (segment (start 114.742081 121.48) (end 117.16 119.062081) (width 0.3) (layer "F.Cu") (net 1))
 (segment (start 117.16 115.08) (end 118.75 113.49) (width 0.3) (layer "F.Cu") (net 1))
 (segment (start 107.782893 131.62) (end 107.34 132.062893) (width 0.3) (layer "F.Cu") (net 1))
 (segment (start 111.64 125.212893) (end 111.64 128.42) (width 0.3) (layer "F.Cu") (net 1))
 (segment (start 112.34 122.68) (end 112.34 124.512893) (width 0.3) (layer "F.Cu") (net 1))
 (segment (start 113.54 108.42) (end 113.64 108.32) (width 0.3) (layer "F.Cu") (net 1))
 (segment (start 113.86 127.95) (end 114.74 127.07) (width 0.3) (layer "F.Cu") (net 1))
 (segment (start 108.44 131.62) (end 107.782893 131.62) (width 0.3) (layer "F.Cu") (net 1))
 (segment (start 107.34 135.02) (end 107.34 141.48) (width 0.3) (layer "F.Cu") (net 1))
 (segment (start 112.34 124.512893) (end 111.64 125.212893) (width 0.3) (layer "F.Cu") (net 1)))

